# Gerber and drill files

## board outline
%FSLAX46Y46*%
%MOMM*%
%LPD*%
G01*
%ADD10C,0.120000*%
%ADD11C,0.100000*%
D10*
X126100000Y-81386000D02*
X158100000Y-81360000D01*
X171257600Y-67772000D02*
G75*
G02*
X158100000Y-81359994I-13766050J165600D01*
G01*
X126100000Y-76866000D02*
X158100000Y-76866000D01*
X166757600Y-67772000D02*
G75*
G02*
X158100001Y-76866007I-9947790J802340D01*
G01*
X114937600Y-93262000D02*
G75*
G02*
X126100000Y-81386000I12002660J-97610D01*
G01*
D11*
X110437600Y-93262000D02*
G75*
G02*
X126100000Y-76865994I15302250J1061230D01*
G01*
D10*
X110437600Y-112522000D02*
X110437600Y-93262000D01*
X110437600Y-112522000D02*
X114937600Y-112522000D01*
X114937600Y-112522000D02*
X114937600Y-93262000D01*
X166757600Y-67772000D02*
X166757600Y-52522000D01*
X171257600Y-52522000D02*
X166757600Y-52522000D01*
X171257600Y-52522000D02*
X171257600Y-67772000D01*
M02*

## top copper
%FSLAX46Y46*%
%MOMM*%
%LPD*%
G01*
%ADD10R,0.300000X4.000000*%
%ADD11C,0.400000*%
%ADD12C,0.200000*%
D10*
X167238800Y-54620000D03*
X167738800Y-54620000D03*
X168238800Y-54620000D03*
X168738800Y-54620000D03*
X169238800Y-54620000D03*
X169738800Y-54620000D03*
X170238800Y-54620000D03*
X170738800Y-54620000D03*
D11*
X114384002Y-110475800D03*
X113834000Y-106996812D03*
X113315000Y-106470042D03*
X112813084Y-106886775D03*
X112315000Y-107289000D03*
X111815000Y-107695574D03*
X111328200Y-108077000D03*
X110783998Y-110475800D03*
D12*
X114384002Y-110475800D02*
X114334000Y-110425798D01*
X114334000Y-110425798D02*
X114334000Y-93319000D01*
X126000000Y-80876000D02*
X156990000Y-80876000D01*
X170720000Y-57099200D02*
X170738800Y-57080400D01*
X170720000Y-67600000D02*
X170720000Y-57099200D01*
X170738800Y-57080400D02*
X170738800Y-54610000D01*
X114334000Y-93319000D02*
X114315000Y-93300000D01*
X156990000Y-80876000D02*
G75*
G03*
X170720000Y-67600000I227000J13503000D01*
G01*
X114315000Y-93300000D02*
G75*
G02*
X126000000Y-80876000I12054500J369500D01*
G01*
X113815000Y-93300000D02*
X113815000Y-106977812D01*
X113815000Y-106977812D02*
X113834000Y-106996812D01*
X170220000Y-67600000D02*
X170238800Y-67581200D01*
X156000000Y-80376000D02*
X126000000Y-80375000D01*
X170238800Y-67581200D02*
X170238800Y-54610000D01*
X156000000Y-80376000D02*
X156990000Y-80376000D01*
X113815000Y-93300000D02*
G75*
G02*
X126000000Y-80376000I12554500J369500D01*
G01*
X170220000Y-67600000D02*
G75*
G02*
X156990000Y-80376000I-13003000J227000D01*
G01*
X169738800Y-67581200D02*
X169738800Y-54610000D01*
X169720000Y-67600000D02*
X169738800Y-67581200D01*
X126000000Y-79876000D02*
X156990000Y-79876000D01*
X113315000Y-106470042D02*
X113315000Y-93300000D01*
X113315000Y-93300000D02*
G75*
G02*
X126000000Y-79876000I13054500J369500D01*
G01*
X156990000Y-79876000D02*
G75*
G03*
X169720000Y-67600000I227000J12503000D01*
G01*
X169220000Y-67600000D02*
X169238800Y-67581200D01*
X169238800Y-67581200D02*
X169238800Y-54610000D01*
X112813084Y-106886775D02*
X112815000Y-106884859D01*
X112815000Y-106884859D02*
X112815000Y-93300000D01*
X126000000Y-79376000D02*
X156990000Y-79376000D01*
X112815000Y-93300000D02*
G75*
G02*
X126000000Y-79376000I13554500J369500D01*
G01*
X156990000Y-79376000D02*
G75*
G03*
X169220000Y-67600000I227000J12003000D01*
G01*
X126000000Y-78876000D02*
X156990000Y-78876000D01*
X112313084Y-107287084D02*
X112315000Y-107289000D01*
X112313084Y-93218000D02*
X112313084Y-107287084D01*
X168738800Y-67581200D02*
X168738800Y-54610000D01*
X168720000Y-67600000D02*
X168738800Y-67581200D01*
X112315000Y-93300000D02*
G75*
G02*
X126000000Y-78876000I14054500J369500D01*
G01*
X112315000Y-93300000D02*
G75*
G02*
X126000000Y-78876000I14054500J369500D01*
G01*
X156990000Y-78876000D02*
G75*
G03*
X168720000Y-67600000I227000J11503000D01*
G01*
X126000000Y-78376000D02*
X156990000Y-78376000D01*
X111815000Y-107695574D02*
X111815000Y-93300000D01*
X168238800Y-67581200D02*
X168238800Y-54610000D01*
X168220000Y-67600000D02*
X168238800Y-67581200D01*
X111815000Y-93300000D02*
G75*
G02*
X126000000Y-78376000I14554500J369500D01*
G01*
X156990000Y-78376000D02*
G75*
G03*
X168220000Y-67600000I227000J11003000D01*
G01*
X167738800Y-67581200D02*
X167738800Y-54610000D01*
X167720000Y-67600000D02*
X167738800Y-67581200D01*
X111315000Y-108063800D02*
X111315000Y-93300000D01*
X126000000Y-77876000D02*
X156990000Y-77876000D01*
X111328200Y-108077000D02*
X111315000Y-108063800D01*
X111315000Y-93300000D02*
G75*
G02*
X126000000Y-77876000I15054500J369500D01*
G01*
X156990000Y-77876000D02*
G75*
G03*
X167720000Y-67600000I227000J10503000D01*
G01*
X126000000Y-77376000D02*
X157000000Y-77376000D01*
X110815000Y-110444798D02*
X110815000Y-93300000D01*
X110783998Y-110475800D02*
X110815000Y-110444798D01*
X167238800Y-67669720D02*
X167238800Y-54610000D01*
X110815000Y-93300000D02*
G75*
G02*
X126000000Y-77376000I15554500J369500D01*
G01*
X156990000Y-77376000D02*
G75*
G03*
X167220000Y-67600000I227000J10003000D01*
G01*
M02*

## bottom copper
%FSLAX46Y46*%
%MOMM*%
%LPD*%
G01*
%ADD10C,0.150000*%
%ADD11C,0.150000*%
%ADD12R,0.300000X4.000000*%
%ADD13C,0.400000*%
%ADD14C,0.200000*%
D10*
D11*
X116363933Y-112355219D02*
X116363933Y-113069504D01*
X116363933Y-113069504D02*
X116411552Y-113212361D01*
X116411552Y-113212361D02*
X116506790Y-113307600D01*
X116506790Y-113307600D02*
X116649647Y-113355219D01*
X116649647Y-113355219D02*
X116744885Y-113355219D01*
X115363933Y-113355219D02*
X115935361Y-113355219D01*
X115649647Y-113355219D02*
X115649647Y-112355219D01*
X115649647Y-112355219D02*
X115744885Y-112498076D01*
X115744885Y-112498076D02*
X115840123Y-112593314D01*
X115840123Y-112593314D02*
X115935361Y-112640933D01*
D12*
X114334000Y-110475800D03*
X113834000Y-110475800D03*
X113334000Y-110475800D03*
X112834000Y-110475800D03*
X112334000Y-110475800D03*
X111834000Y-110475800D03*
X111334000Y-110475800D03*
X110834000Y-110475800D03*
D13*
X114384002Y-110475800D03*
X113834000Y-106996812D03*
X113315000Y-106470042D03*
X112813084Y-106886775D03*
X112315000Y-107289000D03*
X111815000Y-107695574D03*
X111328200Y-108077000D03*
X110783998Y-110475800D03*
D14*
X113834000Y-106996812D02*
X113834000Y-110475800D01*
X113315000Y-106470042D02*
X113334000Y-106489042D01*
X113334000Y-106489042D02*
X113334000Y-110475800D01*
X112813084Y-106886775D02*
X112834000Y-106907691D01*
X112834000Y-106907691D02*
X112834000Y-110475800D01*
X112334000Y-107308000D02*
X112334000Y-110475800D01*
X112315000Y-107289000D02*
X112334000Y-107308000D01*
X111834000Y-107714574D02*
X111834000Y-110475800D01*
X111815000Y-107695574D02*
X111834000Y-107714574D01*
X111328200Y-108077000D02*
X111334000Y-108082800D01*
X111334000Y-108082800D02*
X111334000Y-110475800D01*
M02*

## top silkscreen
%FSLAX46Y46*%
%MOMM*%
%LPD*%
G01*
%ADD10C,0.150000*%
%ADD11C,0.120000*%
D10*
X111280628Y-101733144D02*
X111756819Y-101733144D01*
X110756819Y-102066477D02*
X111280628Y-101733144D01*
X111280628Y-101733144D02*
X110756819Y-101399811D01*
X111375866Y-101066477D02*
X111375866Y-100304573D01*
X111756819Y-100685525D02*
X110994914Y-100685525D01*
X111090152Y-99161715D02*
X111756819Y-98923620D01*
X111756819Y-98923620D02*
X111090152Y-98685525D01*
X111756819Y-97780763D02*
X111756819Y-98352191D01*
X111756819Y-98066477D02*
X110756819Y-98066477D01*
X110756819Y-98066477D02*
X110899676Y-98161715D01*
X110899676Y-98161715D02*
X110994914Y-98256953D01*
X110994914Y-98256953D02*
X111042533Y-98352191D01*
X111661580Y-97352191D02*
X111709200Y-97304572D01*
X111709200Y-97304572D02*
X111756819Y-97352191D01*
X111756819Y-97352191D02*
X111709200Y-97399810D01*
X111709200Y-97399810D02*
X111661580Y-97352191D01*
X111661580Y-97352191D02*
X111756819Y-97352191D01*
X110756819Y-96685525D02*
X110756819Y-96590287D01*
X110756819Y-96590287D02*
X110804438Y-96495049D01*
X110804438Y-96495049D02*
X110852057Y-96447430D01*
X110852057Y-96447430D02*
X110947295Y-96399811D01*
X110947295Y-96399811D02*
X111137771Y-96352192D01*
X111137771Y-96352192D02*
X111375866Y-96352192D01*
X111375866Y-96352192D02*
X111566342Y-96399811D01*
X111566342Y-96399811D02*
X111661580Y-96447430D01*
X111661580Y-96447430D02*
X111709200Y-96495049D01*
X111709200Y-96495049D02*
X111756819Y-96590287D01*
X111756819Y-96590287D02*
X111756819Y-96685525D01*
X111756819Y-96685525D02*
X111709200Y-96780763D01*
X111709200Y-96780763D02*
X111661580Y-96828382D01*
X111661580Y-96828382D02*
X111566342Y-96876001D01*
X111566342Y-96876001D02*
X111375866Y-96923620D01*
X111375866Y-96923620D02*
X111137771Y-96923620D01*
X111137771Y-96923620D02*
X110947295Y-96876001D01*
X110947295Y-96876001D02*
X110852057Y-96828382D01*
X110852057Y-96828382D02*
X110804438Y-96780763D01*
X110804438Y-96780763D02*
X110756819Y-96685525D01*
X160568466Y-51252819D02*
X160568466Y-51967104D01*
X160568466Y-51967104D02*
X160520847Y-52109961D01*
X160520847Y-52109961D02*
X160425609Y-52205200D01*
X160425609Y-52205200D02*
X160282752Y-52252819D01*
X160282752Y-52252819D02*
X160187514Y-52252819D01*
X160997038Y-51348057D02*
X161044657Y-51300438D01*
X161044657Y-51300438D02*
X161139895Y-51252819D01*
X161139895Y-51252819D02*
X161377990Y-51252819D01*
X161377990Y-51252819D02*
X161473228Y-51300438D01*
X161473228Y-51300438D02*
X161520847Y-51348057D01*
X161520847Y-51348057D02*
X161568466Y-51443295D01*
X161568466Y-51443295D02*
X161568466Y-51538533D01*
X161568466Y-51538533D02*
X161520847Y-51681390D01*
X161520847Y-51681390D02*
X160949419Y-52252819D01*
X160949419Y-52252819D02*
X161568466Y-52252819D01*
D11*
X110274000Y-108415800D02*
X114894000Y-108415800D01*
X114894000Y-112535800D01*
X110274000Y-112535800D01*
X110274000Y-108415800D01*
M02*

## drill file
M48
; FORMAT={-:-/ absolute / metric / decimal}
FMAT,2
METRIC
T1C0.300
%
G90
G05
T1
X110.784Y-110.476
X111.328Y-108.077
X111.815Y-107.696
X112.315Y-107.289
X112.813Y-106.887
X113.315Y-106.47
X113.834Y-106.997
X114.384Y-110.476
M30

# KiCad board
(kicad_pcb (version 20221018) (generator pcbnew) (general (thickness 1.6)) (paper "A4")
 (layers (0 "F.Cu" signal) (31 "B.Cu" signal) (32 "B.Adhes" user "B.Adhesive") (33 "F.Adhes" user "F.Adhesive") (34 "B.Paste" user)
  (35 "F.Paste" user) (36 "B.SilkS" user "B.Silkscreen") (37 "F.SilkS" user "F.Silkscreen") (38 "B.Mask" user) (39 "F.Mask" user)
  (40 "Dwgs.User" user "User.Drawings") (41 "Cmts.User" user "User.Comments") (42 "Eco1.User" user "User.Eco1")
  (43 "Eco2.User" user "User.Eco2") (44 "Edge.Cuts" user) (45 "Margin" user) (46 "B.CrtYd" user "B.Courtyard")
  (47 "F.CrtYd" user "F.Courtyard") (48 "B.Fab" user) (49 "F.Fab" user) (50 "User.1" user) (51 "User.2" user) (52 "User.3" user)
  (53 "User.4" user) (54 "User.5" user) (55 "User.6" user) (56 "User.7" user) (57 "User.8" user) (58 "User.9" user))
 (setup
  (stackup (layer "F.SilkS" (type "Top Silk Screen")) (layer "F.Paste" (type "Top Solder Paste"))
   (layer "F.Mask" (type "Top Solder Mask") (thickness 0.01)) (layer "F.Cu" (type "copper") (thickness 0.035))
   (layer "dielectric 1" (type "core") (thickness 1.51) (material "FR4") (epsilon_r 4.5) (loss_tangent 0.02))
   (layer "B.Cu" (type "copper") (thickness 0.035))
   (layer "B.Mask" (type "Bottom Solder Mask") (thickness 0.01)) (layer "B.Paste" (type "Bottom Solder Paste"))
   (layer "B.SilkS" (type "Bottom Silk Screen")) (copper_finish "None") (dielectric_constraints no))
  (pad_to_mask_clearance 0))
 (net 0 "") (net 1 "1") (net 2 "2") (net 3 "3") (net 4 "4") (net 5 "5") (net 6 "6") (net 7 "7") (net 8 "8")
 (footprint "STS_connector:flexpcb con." (layer "F.Cu") (at 166.7388 56.62)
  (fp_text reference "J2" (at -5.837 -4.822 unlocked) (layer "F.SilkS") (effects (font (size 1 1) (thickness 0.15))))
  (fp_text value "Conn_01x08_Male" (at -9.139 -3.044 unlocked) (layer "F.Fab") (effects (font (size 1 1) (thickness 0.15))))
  (pad "1" smd rect (at 0.5 -2) (size 0.3 4) (layers "F.Cu" "F.Paste" "F.Mask") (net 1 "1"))
  (pad "2" smd rect (at 1 -2) (size 0.3 4) (layers "F.Cu" "F.Paste" "F.Mask") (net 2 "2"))
  (pad "3" smd rect (at 1.5 -2) (size 0.3 4) (layers "F.Cu" "F.Paste" "F.Mask") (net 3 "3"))
  (pad "4" smd rect (at 2 -2) (size 0.3 4) (layers "F.Cu" "F.Paste" "F.Mask") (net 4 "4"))
  (pad "5" smd rect (at 2.5 -2) (size 0.3 4) (layers "F.Cu" "F.Paste" "F.Mask") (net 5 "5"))
  (pad "6" smd rect (at 3 -2) (size 0.3 4) (layers "F.Cu" "F.Paste" "F.Mask") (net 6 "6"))
  (pad "7" smd rect (at 3.5 -2) (size 0.3 4) (layers "F.Cu" "F.Paste" "F.Mask") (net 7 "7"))
  (pad "8" smd rect (at 4 -2) (size 0.3 4) (layers "F.Cu" "F.Paste" "F.Mask") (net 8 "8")))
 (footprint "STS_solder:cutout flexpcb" (layer "F.Cu") (at 110.4376 112.522)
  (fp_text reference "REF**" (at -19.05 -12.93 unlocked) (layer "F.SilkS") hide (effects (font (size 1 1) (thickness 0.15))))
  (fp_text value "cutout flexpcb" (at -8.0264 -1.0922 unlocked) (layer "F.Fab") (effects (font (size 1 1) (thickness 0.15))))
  (fp_line (start 0 0) (end 0 -19.26) (stroke (width 0.12) (type solid)) (layer "Edge.Cuts"))
  (fp_line (start 0 0) (end 4.5 0) (stroke (width 0.12) (type solid)) (layer "Edge.Cuts"))
  (fp_line (start 4.5 0) (end 4.5 -19.26) (stroke (width 0.12) (type solid)) (layer "Edge.Cuts"))
  (fp_line (start 56.32 -44.75) (end 56.32 -60) (stroke (width 0.12) (type solid)) (layer "Edge.Cuts"))
  (fp_line (start 60.82 -60) (end 56.32 -60) (stroke (width 0.12) (type solid)) (layer "Edge.Cuts"))
  (fp_line (start 60.82 -60) (end 60.82 -44.75) (stroke (width 0.12) (type solid)) (layer "Edge.Cuts")))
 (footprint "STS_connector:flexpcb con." (layer "B.Cu") (at 114.834 112.4758 180)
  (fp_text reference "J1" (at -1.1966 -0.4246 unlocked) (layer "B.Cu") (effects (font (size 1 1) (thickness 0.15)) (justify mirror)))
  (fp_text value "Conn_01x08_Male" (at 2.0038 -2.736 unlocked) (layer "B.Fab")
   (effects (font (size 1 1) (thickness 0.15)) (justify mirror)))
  (fp_rect (start -0.06 -0.06) (end 4.56 4.06) (stroke (width 0.12) (type solid)) (fill none) (layer "F.SilkS"))
  (pad "1" smd rect (at 0.5 2 180) (size 0.3 4) (layers "B.Cu" "B.Paste" "B.Mask") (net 8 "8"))
  (pad "2" smd rect (at 1 2 180) (size 0.3 4) (layers "B.Cu" "B.Paste" "B.Mask") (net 7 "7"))
  (pad "3" smd rect (at 1.5 2 180) (size 0.3 4) (layers "B.Cu" "B.Paste" "B.Mask") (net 6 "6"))
  (pad "4" smd rect (at 2 2 180) (size 0.3 4) (layers "B.Cu" "B.Paste" "B.Mask") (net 5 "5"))
  (pad "5" smd rect (at 2.5 2 180) (size 0.3 4) (layers "B.Cu" "B.Paste" "B.Mask") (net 4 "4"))
  (pad "6" smd rect (at 3 2 180) (size 0.3 4) (layers "B.Cu" "B.Paste" "B.Mask") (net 3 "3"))
  (pad "7" smd rect (at 3.5 2 180) (size 0.3 4) (layers "B.Cu" "B.Paste" "B.Mask") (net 2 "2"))
  (pad "8" smd rect (at 4 2 180) (size 0.3 4) (layers "B.Cu" "B.Paste" "B.Mask") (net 1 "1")))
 (gr_line (start 126.1 81.386) (end 158.1 81.36) (stroke (width 0.12) (type solid)) (layer "Edge.Cuts"))
 (gr_arc (start 171.2576 67.772) (mid 167.381696 77.183282) (end 158.1 81.36) (stroke (width 0.12) (type solid)) (layer "Edge.Cuts"))
 (gr_line (start 126.1 76.866) (end 158.1 76.866) (stroke (width 0.12) (type solid)) (layer "Edge.Cuts"))
 (gr_arc (start 166.7576 67.772) (mid 164.038106 73.85108) (end 158.1 76.866) (stroke (width 0.12) (type solid)) (layer "Edge.Cuts"))
 (gr_arc (start 114.9376 93.262) (mid 118.194118 85.139003) (end 126.1 81.386) (stroke (width 0.12) (type solid)) (layer "Edge.Cuts"))
 (gr_arc (start 110.4376 93.262) (mid 114.64824 81.605434) (end 126.1 76.866) (stroke (width 0.1) (type default)) (layer "Edge.Cuts"))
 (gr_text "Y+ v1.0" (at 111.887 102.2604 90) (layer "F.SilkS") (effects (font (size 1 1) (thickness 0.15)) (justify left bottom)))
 (segment (start 114.384002 110.4758) (end 114.334 110.425798) (width 0.2) (layer "F.Cu") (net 8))
 (segment (start 114.334 110.425798) (end 114.334 93.319) (width 0.2) (layer "F.Cu") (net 8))
 (segment (start 126 80.876) (end 156.99 80.876) (width 0.2) (layer "F.Cu") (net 8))
 (segment (start 170.72 57.0992) (end 170.7388 57.0804) (width 0.2) (layer "F.Cu") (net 8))
 (segment (start 170.72 67.6) (end 170.72 57.0992) (width 0.2) (layer "F.Cu") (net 8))
 (segment (start 170.7388 57.0804) (end 170.7388 54.61) (width 0.2) (layer "F.Cu") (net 8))
 (segment (start 114.334 93.319) (end 114.315 93.3) (width 0.2) (layer "F.Cu") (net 8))
 (via (at 114.384002 110.4758) (size 0.4) (drill 0.3) (layers "F.Cu" "B.Cu") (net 8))
 (arc (start 156.99 80.876) (mid 166.60455 77.081577) (end 170.72 67.6) (width 0.2) (layer "F.Cu") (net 8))
 (arc (start 114.315 93.3) (mid 117.584405 84.667957) (end 126 80.876) (width 0.2) (layer "F.Cu") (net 8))
 (segment (start 113.815 93.3) (end 113.815 106.977812) (width 0.2) (layer "F.Cu") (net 7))
 (segment (start 113.815 106.977812) (end 113.834 106.996812) (width 0.2) (layer "F.Cu") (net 7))
 (segment (start 170.22 67.6) (end 170.2388 67.5812) (width 0.2) (layer "F.Cu") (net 7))
 (segment (start 156 80.376) (end 126 80.375) (width 0.2) (layer "F.Cu") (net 7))
 (segment (start 170.2388 67.5812) (end 170.2388 54.61) (width 0.2) (layer "F.Cu") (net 7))
 (segment (start 156 80.376) (end 156.99 80.376) (width 0.2) (layer "F.Cu") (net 7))
 (via (at 113.834 106.996812) (size 0.4) (drill 0.3) (layers "F.Cu" "B.Cu") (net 7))
 (arc (start 113.815 93.3) (mid 117.230852 84.314404) (end 126 80.376) (width 0.2) (layer "F.Cu") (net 7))
 (arc (start 170.22 67.6) (mid 166.250997 76.728023) (end 156.99 80.376) (width 0.2) (layer "F.Cu") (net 7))
 (segment (start 113.834 106.996812) (end 113.834 110.4758) (width 0.2) (layer "B.Cu") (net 7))
 (segment (start 169.7388 67.5812) (end 169.7388 54.61) (width 0.2) (layer "F.Cu") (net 6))
 (segment (start 169.72 67.6) (end 169.7388 67.5812) (width 0.2) (layer "F.Cu") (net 6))
 (segment (start 126 79.876) (end 156.99 79.876) (width 0.2) (layer "F.Cu") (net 6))
 (segment (start 113.315 106.470042) (end 113.315 93.3) (width 0.2) (layer "F.Cu") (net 6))
 (via (at 113.315 106.470042) (size 0.4) (drill 0.3) (layers "F.Cu" "B.Cu") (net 6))
 (arc (start 113.315 93.3) (mid 116.877299 83.96085) (end 126 79.876) (width 0.2) (layer "F.Cu") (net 6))
 (arc (start 156.99 79.876) (mid 165.897443 76.374469) (end 169.72 67.6) (width 0.2) (layer "F.Cu") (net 6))
 (segment (start 113.315 106.470042) (end 113.334 106.489042) (width 0.2) (layer "B.Cu") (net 6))
 (segment (start 113.334 106.489042) (end 113.334 110.4758) (width 0.2) (layer "B.Cu") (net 6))
 (segment (start 169.22 67.6) (end 169.2388 67.5812) (width 0.2) (layer "F.Cu") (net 5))
 (segment (start 169.2388 67.5812) (end 169.2388 54.61) (width 0.2) (layer "F.Cu") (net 5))
 (segment (start 112.813084 106.886775) (end 112.815 106.884859) (width 0.2) (layer "F.Cu") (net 5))
 (segment (start 112.815 106.884859) (end 112.815 93.3) (width 0.2) (layer "F.Cu") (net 5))
 (segment (start 126 79.376) (end 156.99 79.376) (width 0.2) (layer "F.Cu") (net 5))
 (via (at 112.813084 106.886775) (size 0.4) (drill 0.3) (layers "F.Cu" "B.Cu") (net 5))
 (arc (start 112.815 93.3) (mid 116.523745 83.607297) (end 126 79.376) (width 0.2) (layer "F.Cu") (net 5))
 (arc (start 156.99 79.376) (mid 165.54389 76.020917) (end 169.22 67.6) (width 0.2) (layer "F.Cu") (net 5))
 (segment (start 112.813084 106.886775) (end 112.834 106.907691) (width 0.2) (layer "B.Cu") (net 5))
 (segment (start 112.834 106.907691) (end 112.834 110.4758) (width 0.2) (layer "B.Cu") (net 5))
 (segment (start 126 78.876) (end 156.99 78.876) (width 0.2) (layer "F.Cu") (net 4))
 (segment (start 112.313084 107.287084) (end 112.315 107.289) (width 0.2) (layer "F.Cu") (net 4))
 (segment (start 112.313084 93.218) (end 112.313084 107.287084) (width 0.2) (layer "F.Cu") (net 4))
 (segment (start 168.7388 67.5812) (end 168.7388 54.61) (width 0.2) (layer "F.Cu") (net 4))
 (segment (start 168.72 67.6) (end 168.7388 67.5812) (width 0.2) (layer "F.Cu") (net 4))
 (via (at 112.315 107.289) (size 0.4) (drill 0.3) (layers "F.Cu" "B.Cu") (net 4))
 (arc (start 112.315 93.3) (mid 116.170192 83.253744) (end 126 78.876) (width 0.2) (layer "F.Cu") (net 4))
 (arc (start 112.315 93.3) (mid 116.170192 83.253744) (end 126 78.876) (width 0.2) (layer "F.Cu") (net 4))
 (arc (start 156.99 78.876) (mid 165.190336 75.667363) (end 168.72 67.6) (width 0.2) (layer "F.Cu") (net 4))
 (segment (start 112.334 107.308) (end 112.334 110.4758) (width 0.2) (layer "B.Cu") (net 4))
 (segment (start 112.315 107.289) (end 112.334 107.308) (width 0.2) (layer "B.Cu") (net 4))
 (segment (start 126 78.376) (end 156.99 78.376) (width 0.2) (layer "F.Cu") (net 3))
 (segment (start 111.815 107.695574) (end 111.815 93.3) (width 0.2) (layer "F.Cu") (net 3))
 (segment (start 168.2388 67.5812) (end 168.2388 54.61) (width 0.2) (layer "F.Cu") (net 3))
 (segment (start 168.22 67.6) (end 168.2388 67.5812) (width 0.2) (layer "F.Cu") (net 3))
 (via (at 111.815 107.695574) (size 0.4) (drill 0.3) (layers "F.Cu" "B.Cu") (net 3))
 (arc (start 111.815 93.3) (mid 115.816638 82.90019) (end 126 78.376) (width 0.2) (layer "F.Cu") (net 3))
 (arc (start 156.99 78.376) (mid 164.836783 75.313809) (end 168.22 67.6) (width 0.2) (layer "F.Cu") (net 3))
 (segment (start 111.834 107.714574) (end 111.834 110.4758) (width 0.2) (layer "B.Cu") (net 3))
 (segment (start 111.815 107.695574) (end 111.834 107.714574) (width 0.2) (layer "B.Cu") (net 3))
 (segment (start 167.7388 67.5812) (end 167.7388 54.61) (width 0.2) (layer "F.Cu") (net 2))
 (segment (start 167.72 67.6) (end 167.7388 67.5812) (width 0.2) (layer "F.Cu") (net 2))
 (segment (start 111.315 108.0638) (end 111.315 93.3) (width 0.2) (layer "F.Cu") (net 2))
 (segment (start 126 77.876) (end 156.99 77.876) (width 0.2) (layer "F.Cu") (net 2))
 (segment (start 111.3282 108.077) (end 111.315 108.0638) (width 0.2) (layer "F.Cu") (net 2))
 (via (at 111.3282 108.077) (size 0.4) (drill 0.3) (layers "F.Cu" "B.Cu") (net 2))
 (arc (start 111.315 93.3) (mid 115.463085 82.546637) (end 126 77.876) (width 0.2) (layer "F.Cu") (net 2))
 (arc (start 156.99 77.876) (mid 164.483229 74.960256) (end 167.72 67.6) (width 0.2) (layer "F.Cu") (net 2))
 (segment (start 111.3282 108.077) (end 111.334 108.0828) (width 0.2) (layer "B.Cu") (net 2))
 (segment (start 111.334 108.0828) (end 111.334 110.4758) (width 0.2) (layer "B.Cu") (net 2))
 (segment (start 126 77.376) (end 157 77.376) (width 0.2) (layer "F.Cu") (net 1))
 (segment (start 110.815 110.444798) (end 110.815 93.3) (width 0.2) (layer "F.Cu") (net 1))
 (segment (start 110.783998 110.4758) (end 110.815 110.444798) (width 0.2) (layer "F.Cu") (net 1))
 (segment (start 167.2388 67.66972) (end 167.2388 54.61) (width 0.2) (layer "F.Cu") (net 1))
 (via (at 110.783998 110.4758) (size 0.4) (drill 0.3) (layers "F.Cu" "B.Cu") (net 1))
 (arc (start 110.815 93.3) (mid 115.109532 82.193084) (end 126 77.376) (width 0.2) (layer "F.Cu") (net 1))
 (arc (start 156.99 77.376) (mid 164.129676 74.606702) (end 167.22 67.6) (width 0.2) (layer "F.Cu") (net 1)))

